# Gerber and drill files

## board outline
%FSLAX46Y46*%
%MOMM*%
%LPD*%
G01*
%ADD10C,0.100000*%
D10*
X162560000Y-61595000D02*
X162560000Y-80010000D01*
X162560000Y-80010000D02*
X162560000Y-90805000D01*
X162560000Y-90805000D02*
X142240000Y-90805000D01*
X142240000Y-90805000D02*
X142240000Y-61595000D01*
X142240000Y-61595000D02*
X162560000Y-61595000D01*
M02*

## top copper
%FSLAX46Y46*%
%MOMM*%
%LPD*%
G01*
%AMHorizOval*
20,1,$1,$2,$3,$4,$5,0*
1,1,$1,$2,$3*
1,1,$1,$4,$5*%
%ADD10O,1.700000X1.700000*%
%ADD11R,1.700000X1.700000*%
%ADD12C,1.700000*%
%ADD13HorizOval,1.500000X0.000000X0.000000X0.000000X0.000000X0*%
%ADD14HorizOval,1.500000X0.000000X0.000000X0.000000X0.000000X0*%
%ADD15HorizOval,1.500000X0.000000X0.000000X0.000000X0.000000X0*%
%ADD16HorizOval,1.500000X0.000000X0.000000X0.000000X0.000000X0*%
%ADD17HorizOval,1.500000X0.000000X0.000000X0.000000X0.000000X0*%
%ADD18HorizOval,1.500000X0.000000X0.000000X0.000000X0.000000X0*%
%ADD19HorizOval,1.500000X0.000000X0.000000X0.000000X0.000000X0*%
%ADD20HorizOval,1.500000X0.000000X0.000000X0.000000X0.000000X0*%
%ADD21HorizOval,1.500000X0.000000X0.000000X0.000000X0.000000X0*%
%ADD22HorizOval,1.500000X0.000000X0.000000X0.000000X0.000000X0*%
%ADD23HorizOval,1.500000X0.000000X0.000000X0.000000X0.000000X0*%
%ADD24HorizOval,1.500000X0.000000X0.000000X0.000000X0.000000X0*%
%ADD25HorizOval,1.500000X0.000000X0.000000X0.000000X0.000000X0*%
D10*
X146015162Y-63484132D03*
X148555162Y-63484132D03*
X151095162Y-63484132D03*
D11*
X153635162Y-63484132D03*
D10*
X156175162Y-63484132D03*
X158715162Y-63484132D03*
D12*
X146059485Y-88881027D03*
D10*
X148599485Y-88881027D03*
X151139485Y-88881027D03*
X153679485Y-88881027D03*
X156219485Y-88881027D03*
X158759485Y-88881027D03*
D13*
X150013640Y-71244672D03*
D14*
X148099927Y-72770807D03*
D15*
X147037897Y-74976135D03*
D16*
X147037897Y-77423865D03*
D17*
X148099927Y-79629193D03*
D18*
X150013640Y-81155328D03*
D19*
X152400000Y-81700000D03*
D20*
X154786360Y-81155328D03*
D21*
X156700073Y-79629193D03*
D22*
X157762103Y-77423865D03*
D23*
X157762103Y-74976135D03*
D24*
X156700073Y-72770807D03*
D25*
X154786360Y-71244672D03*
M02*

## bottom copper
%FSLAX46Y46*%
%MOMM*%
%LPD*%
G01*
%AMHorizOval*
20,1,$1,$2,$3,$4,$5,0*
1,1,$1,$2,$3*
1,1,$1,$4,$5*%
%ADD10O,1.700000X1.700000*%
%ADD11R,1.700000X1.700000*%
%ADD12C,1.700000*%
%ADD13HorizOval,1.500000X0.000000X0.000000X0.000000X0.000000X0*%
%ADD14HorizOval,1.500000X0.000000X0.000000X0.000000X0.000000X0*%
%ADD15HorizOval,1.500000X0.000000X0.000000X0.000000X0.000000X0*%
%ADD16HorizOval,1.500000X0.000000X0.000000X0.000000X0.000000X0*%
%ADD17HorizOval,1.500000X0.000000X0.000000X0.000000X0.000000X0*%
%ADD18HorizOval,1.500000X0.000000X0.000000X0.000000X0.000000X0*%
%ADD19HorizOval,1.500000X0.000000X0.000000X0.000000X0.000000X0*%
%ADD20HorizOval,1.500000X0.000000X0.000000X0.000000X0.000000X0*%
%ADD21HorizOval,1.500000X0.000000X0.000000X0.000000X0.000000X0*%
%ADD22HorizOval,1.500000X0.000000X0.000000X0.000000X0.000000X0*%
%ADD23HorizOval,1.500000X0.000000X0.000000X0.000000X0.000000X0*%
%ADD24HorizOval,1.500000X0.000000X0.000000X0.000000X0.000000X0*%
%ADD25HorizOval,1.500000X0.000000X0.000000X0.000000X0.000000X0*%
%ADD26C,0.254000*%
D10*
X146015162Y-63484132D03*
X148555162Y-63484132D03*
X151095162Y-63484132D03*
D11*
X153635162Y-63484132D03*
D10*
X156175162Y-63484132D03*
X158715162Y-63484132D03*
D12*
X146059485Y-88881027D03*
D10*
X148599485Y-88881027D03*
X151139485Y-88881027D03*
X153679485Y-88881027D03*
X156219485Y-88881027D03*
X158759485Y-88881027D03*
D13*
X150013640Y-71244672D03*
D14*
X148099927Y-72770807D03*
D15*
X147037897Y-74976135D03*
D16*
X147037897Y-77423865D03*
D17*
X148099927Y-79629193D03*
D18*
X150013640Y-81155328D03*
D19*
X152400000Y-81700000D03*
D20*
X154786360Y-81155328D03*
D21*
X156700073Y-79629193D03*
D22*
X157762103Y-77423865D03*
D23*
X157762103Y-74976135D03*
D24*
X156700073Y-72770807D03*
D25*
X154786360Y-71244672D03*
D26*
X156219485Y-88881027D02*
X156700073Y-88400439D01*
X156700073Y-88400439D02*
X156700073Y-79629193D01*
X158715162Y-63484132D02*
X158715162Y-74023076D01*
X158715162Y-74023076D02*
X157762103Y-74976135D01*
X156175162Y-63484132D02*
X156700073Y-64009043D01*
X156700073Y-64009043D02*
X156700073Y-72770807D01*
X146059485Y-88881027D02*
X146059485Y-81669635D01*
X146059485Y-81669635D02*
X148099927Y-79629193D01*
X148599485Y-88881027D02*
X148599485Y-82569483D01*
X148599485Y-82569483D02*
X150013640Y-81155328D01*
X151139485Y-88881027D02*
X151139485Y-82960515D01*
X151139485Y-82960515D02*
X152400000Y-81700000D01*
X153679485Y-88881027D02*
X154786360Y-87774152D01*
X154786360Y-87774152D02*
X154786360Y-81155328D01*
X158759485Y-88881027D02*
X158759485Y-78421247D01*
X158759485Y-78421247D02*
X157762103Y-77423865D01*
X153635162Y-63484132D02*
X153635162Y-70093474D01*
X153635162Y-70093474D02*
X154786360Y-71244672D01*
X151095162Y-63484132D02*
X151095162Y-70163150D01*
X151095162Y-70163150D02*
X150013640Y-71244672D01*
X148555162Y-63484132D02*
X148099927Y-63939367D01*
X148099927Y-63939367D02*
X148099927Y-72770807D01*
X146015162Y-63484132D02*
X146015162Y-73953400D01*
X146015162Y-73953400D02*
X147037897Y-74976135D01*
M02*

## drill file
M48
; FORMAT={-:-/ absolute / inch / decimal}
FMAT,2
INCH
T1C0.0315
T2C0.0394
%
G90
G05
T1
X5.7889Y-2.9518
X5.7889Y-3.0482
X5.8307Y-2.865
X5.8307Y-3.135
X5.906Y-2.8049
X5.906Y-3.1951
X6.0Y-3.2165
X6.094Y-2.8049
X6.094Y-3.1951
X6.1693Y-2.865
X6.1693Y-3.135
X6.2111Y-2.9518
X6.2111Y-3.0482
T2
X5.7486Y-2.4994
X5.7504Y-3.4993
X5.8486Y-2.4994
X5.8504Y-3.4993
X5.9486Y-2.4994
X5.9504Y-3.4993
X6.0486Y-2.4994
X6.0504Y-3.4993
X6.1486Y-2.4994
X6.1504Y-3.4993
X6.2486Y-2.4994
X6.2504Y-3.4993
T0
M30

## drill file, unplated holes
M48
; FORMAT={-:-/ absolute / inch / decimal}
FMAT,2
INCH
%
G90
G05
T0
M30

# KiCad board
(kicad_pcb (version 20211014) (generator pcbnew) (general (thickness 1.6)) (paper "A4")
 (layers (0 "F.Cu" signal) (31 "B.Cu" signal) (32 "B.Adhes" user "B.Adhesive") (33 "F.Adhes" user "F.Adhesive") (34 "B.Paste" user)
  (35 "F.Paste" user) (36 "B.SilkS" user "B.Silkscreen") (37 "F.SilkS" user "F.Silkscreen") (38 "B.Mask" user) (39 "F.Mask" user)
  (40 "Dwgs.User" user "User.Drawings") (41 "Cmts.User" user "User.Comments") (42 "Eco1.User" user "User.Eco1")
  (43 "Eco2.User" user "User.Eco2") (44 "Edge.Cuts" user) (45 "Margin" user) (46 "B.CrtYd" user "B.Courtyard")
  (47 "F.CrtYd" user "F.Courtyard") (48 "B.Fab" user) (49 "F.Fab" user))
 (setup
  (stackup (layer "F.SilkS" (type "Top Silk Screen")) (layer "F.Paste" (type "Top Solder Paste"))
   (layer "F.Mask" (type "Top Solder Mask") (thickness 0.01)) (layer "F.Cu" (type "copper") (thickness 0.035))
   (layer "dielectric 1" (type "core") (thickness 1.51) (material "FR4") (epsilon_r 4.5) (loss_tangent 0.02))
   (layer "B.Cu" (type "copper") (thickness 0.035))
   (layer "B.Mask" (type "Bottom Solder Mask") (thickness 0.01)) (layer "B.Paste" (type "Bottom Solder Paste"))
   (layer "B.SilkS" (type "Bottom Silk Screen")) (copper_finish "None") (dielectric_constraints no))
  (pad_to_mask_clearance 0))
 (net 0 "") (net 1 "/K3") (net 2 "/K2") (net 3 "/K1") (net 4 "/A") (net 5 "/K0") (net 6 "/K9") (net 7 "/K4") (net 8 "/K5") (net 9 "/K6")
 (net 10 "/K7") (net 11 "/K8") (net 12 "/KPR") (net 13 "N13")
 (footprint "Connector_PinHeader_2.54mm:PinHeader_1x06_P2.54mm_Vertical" (layer "F.Cu") (at 146.015162 63.484132 90)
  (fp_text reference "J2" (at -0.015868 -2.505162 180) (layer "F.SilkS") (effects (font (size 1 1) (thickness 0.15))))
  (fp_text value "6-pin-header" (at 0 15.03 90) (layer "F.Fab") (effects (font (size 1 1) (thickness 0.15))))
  (pad "1" thru_hole oval (at 0 0 90) (size 1.7 1.7) (drill 1) (layers *.Cu *.Mask) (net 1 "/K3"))
  (pad "2" thru_hole oval (at 0 2.54 90) (size 1.7 1.7) (drill 1) (layers *.Cu *.Mask) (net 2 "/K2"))
  (pad "3" thru_hole oval (at 0 5.08 90) (size 1.7 1.7) (drill 1) (layers *.Cu *.Mask) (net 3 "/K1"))
  (pad "4" thru_hole rect (at 0 7.62 90) (size 1.7 1.7) (drill 1) (layers *.Cu *.Mask) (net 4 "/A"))
  (pad "5" thru_hole oval (at 0 10.16 90) (size 1.7 1.7) (drill 1) (layers *.Cu *.Mask) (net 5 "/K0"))
  (pad "6" thru_hole oval (at 0 12.7 90) (size 1.7 1.7) (drill 1) (layers *.Cu *.Mask) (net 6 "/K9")))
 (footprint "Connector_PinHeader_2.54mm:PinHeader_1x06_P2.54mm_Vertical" (layer "F.Cu") (at 146.059485 88.881027 90)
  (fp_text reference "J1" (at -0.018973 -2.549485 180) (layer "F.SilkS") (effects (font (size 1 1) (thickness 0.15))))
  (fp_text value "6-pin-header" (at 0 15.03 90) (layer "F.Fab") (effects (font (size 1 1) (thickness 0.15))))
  (pad "1" thru_hole circle (at 0 0 90) (size 1.7 1.7) (drill 1) (layers *.Cu *.Mask) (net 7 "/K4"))
  (pad "2" thru_hole oval (at 0 2.54 90) (size 1.7 1.7) (drill 1) (layers *.Cu *.Mask) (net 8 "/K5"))
  (pad "3" thru_hole oval (at 0 5.08 90) (size 1.7 1.7) (drill 1) (layers *.Cu *.Mask) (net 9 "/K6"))
  (pad "4" thru_hole oval (at 0 7.62 90) (size 1.7 1.7) (drill 1) (layers *.Cu *.Mask) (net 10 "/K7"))
  (pad "5" thru_hole oval (at 0 10.16 90) (size 1.7 1.7) (drill 1) (layers *.Cu *.Mask) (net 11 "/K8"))
  (pad "6" thru_hole oval (at 0 12.7 90) (size 1.7 1.7) (drill 1) (layers *.Cu *.Mask) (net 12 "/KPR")))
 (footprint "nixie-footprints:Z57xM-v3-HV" (layer "F.Cu") (at 152.4 76.2)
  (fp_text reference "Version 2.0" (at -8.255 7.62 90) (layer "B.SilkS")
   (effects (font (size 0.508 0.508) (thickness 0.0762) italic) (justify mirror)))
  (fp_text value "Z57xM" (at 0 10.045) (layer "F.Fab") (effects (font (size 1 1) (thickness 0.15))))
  (pad "1" thru_hole oval (at -2.38636 -4.955328 51.414) (size 1.5 1.5) (drill 0.8) (layers *.Cu *.Mask) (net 3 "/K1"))
  (pad "2" thru_hole oval (at -4.300073 -3.429193 77.128) (size 1.5 1.5) (drill 0.8) (layers *.Cu *.Mask) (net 2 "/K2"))
  (pad "3" thru_hole oval (at -5.362103 -1.223865 102.842) (size 1.5 1.5) (drill 0.8) (layers *.Cu *.Mask) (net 1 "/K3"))
  (pad "4" thru_hole oval (at -5.362103 1.223865 128.556) (size 1.5 1.5) (drill 0.8) (layers *.Cu *.Mask) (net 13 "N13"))
  (pad "5" thru_hole oval (at -4.300073 3.429193 154.271) (size 1.5 1.5) (drill 0.8) (layers *.Cu *.Mask) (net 7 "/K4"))
  (pad "6" thru_hole oval (at -2.38636 4.955328 179.985) (size 1.5 1.5) (drill 0.8) (layers *.Cu *.Mask) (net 8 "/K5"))
  (pad "7" thru_hole oval (at 0 5.5 205.7) (size 1.5 1.5) (drill 0.8) (layers *.Cu *.Mask) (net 9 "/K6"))
  (pad "8" thru_hole oval (at 2.38636 4.955328 231.414) (size 1.5 1.5) (drill 0.8) (layers *.Cu *.Mask) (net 10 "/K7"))
  (pad "9" thru_hole oval (at 4.300073 3.429193 257.128) (size 1.5 1.5) (drill 0.8) (layers *.Cu *.Mask) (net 11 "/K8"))
  (pad "10" thru_hole oval (at 5.362103 1.223865 282.842) (size 1.5 1.5) (drill 0.8) (layers *.Cu *.Mask) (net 12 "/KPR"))
  (pad "11" thru_hole oval (at 5.362103 -1.223865 308.557) (size 1.5 1.5) (drill 0.8) (layers *.Cu *.Mask) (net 6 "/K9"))
  (pad "12" thru_hole oval (at 4.300073 -3.429193 334.271) (size 1.5 1.5) (drill 0.8) (layers *.Cu *.Mask) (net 5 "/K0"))
  (pad "13" thru_hole oval (at 2.38636 -4.955328 359.985) (size 1.5 1.5) (drill 0.8) (layers *.Cu *.Mask) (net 4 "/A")))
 (gr_line (start 162.56 61.595) (end 162.56 80.01) (layer "Edge.Cuts") (width 0.1))
 (gr_line (start 162.56 80.01) (end 162.56 90.805) (layer "Edge.Cuts") (width 0.1))
 (gr_line (start 162.56 90.805) (end 142.24 90.805) (layer "Edge.Cuts") (width 0.1))
 (gr_line (start 142.24 90.805) (end 142.24 61.595) (layer "Edge.Cuts") (width 0.1))
 (gr_line (start 142.24 61.595) (end 162.56 61.595) (layer "Edge.Cuts") (width 0.1))
 (segment (start 158.759485 78.421247) (end 157.762103 77.423865) (width 0.254) (layer "B.Cu") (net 12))
 (segment (start 158.759485 88.881027) (end 158.759485 78.421247) (width 0.254) (layer "B.Cu") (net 12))
 (segment (start 156.700073 88.400439) (end 156.700073 79.629193) (width 0.254) (layer "B.Cu") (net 11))
 (segment (start 156.219485 88.881027) (end 156.700073 88.400439) (width 0.254) (layer "B.Cu") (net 11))
 (segment (start 153.679485 88.881027) (end 154.78636 87.774152) (width 0.254) (layer "B.Cu") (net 10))
 (segment (start 154.78636 87.774152) (end 154.78636 81.155328) (width 0.254) (layer "B.Cu") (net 10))
 (segment (start 151.139485 82.960515) (end 152.4 81.7) (width 0.254) (layer "B.Cu") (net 9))
 (segment (start 151.139485 88.881027) (end 151.139485 82.960515) (width 0.254) (layer "B.Cu") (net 9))
 (segment (start 148.599485 82.569483) (end 150.01364 81.155328) (width 0.254) (layer "B.Cu") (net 8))
 (segment (start 148.599485 88.881027) (end 148.599485 82.569483) (width 0.254) (layer "B.Cu") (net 8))
 (segment (start 146.059485 88.881027) (end 146.059485 81.669635) (width 0.254) (layer "B.Cu") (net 7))
 (segment (start 146.059485 81.669635) (end 148.099927 79.629193) (width 0.254) (layer "B.Cu") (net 7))
 (segment (start 146.015162 73.9534) (end 147.037897 74.976135) (width 0.254) (layer "B.Cu") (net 1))
 (segment (start 146.015162 63.484132) (end 146.015162 73.9534) (width 0.254) (layer "B.Cu") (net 1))
 (segment (start 148.099927 63.939367) (end 148.099927 72.770807) (width 0.254) (layer "B.Cu") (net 2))
 (segment (start 148.555162 63.484132) (end 148.099927 63.939367) (width 0.254) (layer "B.Cu") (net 2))
 (segment (start 151.095162 63.484132) (end 151.095162 70.16315) (width 0.254) (layer "B.Cu") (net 3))
 (segment (start 151.095162 70.16315) (end 150.01364 71.244672) (width 0.254) (layer "B.Cu") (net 3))
 (segment (start 153.635162 70.093474) (end 154.78636 71.244672) (width 0.254) (layer "B.Cu") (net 4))
 (segment (start 153.635162 63.484132) (end 153.635162 70.093474) (width 0.254) (layer "B.Cu") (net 4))
 (segment (start 156.700073 64.009043) (end 156.700073 72.770807) (width 0.254) (layer "B.Cu") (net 5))
 (segment (start 156.175162 63.484132) (end 156.700073 64.009043) (width 0.254) (layer "B.Cu") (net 5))
 (segment (start 158.715162 74.023076) (end 157.762103 74.976135) (width 0.254) (layer "B.Cu") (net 6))
 (segment (start 158.715162 63.484132) (end 158.715162 74.023076) (width 0.254) (layer "B.Cu") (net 6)))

